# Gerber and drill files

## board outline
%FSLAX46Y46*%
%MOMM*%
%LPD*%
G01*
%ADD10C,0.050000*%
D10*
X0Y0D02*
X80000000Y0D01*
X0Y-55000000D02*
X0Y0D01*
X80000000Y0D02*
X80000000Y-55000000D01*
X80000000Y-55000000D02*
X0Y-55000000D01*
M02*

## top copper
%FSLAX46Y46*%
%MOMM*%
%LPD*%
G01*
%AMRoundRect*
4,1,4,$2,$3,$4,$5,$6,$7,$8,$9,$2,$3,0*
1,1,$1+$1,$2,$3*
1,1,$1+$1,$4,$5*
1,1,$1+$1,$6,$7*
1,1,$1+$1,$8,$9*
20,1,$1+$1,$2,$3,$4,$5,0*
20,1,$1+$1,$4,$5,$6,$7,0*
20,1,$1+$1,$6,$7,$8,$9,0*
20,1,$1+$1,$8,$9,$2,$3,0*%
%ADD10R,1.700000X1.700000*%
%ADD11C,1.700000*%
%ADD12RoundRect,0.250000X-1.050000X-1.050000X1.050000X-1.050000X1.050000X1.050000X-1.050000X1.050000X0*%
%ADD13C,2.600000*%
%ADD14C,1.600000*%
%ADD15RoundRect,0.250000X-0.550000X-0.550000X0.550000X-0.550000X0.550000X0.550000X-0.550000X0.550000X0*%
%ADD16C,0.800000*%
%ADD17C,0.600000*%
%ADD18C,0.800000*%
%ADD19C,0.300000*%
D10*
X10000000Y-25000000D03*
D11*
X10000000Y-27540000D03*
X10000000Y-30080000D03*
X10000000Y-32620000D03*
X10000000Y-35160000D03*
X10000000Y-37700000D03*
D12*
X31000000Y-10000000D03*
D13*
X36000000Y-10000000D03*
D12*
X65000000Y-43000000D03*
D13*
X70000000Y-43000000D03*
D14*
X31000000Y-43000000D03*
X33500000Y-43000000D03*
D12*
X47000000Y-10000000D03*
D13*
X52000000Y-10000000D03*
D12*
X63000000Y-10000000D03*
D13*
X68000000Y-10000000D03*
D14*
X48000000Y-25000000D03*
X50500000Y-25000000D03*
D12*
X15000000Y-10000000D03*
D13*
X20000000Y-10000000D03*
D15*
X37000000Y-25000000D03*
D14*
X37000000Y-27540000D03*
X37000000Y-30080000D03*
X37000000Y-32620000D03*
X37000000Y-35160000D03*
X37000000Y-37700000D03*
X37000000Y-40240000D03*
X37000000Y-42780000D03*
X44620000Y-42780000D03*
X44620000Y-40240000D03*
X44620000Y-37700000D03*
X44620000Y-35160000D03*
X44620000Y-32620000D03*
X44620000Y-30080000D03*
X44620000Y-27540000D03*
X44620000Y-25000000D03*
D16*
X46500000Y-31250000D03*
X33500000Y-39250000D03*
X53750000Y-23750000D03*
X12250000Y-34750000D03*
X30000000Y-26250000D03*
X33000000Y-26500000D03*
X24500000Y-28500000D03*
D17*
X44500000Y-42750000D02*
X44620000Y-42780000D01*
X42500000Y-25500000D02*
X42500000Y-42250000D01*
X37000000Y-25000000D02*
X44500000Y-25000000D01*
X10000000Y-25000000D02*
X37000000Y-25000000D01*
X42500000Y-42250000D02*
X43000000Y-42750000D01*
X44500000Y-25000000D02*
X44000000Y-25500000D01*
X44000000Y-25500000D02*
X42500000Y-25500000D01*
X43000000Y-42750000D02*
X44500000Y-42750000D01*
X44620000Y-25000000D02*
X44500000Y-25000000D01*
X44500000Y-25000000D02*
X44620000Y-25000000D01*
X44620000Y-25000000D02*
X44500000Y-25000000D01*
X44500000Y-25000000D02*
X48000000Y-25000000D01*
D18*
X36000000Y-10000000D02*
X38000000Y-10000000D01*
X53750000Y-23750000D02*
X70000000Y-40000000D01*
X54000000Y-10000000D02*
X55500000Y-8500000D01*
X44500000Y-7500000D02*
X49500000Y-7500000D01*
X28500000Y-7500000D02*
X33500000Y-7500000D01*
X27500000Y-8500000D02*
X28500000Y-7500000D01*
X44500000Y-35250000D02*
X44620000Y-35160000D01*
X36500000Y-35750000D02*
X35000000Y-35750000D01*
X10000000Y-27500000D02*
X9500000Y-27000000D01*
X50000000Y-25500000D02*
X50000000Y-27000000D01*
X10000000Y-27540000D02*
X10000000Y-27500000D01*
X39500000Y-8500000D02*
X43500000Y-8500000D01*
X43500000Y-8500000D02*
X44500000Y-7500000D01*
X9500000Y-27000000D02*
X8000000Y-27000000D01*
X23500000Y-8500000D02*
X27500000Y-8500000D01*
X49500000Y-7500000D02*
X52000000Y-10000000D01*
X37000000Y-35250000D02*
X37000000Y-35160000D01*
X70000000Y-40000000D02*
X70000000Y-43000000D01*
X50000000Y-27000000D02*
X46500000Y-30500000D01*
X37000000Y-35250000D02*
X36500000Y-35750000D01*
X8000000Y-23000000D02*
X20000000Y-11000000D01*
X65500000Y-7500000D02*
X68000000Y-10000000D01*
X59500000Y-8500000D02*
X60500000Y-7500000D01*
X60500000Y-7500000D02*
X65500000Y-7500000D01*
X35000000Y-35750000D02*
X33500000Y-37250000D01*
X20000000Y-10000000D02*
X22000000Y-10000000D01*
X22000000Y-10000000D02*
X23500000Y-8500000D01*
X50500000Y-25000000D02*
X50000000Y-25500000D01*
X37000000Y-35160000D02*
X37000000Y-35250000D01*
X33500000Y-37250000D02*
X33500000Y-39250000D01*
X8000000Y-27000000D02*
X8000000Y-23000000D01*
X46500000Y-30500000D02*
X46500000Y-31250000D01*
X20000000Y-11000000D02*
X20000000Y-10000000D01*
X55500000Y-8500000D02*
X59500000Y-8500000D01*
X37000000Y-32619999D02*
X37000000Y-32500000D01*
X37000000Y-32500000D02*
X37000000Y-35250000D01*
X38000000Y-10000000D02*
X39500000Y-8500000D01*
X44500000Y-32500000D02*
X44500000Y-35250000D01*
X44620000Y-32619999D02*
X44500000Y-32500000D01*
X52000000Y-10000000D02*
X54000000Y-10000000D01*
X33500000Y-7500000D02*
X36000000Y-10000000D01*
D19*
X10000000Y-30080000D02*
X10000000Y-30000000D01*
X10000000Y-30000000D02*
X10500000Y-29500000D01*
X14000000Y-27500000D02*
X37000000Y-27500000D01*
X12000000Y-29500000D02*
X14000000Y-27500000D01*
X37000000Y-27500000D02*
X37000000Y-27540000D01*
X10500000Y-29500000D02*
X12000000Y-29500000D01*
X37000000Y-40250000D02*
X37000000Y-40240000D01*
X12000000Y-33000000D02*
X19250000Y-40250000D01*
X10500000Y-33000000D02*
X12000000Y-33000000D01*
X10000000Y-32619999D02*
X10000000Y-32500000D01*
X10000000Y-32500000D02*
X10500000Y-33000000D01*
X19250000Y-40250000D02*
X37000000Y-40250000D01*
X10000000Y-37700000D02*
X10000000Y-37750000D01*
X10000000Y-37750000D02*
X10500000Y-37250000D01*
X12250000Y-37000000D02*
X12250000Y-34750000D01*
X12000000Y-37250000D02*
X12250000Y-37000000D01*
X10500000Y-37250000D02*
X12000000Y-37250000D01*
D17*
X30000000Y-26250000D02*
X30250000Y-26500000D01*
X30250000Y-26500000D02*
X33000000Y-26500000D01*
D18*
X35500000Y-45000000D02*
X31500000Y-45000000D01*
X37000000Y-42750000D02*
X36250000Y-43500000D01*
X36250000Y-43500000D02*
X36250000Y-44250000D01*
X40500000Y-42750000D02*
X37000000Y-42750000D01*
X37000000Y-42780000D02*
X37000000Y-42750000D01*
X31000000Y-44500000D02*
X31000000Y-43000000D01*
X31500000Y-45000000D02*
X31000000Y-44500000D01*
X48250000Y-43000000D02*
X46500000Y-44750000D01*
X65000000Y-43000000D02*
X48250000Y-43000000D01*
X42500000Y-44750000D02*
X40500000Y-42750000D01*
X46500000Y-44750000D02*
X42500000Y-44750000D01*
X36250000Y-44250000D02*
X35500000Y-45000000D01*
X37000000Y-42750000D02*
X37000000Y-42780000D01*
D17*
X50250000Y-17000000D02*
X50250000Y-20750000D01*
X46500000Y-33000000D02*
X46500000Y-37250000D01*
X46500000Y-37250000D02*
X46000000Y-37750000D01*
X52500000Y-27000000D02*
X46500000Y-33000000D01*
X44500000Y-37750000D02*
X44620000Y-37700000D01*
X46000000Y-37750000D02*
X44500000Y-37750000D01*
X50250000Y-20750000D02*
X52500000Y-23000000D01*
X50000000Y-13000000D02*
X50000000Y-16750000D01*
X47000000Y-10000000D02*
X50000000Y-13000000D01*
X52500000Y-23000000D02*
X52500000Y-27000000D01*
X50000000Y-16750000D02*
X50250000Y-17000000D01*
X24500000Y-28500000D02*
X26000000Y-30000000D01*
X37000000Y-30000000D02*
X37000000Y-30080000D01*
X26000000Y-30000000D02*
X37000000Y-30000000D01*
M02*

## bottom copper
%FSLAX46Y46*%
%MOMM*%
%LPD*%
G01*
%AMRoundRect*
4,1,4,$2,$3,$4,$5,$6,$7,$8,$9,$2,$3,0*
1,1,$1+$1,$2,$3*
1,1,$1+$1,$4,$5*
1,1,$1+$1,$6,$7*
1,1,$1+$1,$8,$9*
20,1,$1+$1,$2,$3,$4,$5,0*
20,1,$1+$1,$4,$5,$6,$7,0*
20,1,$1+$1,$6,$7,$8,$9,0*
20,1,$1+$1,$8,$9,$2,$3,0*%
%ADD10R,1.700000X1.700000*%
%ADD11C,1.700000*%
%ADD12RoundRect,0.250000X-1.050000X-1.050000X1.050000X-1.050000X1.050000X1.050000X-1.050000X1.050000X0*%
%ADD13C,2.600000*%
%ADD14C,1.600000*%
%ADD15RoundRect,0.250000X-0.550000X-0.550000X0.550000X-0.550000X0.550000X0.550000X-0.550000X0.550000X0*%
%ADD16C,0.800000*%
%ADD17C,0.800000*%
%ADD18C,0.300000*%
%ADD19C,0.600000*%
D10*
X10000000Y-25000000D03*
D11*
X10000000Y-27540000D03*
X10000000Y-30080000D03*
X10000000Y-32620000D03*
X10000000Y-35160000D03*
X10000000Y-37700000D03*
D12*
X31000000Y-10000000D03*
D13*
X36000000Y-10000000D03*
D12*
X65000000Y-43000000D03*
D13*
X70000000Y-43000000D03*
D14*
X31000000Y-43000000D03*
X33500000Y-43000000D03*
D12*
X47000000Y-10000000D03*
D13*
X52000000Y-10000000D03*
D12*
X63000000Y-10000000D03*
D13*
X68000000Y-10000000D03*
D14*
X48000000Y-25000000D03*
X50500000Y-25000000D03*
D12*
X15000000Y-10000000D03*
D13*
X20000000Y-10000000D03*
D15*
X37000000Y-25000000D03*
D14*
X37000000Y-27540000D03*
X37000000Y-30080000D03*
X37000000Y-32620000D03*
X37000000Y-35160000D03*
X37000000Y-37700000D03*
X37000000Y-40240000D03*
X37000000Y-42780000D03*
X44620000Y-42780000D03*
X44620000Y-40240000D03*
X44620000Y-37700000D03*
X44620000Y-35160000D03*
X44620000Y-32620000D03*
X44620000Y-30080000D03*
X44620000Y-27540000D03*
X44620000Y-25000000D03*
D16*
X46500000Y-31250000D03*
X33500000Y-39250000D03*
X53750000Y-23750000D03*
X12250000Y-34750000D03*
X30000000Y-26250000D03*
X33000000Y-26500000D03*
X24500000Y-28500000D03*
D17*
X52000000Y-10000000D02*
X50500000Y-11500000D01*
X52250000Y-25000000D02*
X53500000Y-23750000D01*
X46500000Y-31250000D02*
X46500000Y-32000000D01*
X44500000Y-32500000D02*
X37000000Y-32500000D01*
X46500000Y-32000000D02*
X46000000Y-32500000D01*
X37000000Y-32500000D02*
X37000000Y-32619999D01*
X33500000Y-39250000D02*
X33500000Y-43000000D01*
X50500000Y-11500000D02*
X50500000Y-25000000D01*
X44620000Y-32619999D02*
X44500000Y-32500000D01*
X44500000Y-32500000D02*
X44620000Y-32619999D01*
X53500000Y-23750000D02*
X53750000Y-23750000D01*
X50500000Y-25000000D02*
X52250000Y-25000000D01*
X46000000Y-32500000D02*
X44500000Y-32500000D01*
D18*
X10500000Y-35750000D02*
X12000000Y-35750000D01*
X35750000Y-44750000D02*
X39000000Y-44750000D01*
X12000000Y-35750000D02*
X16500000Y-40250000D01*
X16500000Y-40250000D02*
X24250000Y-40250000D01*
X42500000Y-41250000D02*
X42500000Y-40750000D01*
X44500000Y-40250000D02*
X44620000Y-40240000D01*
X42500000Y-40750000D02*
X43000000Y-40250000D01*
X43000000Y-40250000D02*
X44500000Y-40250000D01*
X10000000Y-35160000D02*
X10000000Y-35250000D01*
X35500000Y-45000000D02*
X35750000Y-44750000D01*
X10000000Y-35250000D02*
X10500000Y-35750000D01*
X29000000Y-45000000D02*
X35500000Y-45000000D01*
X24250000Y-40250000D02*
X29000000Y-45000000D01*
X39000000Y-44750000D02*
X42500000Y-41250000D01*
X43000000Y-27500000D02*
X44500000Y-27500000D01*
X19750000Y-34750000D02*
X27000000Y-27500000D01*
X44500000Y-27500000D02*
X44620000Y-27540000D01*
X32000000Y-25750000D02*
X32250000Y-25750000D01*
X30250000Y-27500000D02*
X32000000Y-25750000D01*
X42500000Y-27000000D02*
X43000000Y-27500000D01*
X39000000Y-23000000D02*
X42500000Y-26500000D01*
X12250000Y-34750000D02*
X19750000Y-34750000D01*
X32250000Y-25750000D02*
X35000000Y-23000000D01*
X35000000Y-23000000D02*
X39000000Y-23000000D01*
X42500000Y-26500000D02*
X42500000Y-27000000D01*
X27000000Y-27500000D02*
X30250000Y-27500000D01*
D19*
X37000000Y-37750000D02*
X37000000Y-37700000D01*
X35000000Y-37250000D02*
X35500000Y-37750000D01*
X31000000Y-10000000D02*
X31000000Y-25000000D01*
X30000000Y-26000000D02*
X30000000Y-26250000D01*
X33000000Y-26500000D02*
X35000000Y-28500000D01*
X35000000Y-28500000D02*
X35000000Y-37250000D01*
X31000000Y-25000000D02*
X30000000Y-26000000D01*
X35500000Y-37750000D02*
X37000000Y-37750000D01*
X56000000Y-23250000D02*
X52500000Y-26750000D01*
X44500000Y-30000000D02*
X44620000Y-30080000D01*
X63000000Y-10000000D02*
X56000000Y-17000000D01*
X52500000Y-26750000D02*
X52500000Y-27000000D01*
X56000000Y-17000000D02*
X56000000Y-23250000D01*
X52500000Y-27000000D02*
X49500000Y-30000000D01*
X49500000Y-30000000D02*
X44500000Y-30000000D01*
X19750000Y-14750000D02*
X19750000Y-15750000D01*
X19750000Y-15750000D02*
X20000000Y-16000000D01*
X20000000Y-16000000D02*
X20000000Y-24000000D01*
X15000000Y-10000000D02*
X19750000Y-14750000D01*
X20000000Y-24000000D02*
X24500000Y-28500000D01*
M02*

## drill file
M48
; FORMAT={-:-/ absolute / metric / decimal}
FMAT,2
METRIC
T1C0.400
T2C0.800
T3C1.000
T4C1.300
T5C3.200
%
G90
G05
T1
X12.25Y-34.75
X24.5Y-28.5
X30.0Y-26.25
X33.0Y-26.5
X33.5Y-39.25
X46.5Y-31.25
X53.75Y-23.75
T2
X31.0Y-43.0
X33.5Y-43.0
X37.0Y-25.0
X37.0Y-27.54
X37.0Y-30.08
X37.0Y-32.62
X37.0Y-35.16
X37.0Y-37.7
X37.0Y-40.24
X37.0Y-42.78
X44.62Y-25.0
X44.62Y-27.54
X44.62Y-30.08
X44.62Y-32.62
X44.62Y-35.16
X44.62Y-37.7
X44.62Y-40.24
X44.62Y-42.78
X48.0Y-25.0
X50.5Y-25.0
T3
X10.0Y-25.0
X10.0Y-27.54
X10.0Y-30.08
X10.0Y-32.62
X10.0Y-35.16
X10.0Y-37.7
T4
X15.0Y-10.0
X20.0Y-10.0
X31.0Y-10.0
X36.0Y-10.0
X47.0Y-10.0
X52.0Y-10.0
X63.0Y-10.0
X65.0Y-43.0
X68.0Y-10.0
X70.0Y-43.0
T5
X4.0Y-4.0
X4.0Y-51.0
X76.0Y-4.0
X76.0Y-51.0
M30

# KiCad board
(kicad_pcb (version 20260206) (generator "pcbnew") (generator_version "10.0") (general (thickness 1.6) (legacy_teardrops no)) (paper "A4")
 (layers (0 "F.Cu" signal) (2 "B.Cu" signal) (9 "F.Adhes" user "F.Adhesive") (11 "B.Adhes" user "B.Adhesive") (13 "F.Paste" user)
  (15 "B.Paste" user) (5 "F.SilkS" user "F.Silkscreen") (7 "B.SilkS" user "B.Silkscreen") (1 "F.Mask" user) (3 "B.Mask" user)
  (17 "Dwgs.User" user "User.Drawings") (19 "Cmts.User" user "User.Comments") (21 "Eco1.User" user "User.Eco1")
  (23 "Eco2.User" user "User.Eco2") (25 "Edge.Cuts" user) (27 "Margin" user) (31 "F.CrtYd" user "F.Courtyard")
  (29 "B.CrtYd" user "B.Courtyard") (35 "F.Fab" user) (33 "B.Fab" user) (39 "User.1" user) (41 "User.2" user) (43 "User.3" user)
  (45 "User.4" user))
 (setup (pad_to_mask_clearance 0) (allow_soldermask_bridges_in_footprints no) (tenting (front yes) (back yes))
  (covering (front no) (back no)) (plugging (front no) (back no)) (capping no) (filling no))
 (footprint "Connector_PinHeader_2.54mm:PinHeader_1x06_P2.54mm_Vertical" (layer "F.Cu") (at 10 25)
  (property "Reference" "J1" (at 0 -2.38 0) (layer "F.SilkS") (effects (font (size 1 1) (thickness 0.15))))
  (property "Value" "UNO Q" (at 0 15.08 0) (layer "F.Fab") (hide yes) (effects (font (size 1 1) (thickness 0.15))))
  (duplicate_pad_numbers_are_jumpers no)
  (pad "1" thru_hole rect (at 0 0) (size 1.7 1.7) (drill 1) (layers "*.Cu" "*.Mask") (remove_unused_layers no) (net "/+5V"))
  (pad "2" thru_hole circle (at 0 2.54) (size 1.7 1.7) (drill 1) (layers "*.Cu" "*.Mask") (remove_unused_layers no) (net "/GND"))
  (pad "3" thru_hole circle (at 0 5.08) (size 1.7 1.7) (drill 1) (layers "*.Cu" "*.Mask") (remove_unused_layers no) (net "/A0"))
  (pad "4" thru_hole circle (at 0 7.62) (size 1.7 1.7) (drill 1) (layers "*.Cu" "*.Mask") (remove_unused_layers no) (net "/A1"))
  (pad "5" thru_hole circle (at 0 10.16) (size 1.7 1.7) (drill 1) (layers "*.Cu" "*.Mask") (remove_unused_layers no) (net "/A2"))
  (pad "6" thru_hole circle (at 0 12.7) (size 1.7 1.7) (drill 1) (layers "*.Cu" "*.Mask") (remove_unused_layers no) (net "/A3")))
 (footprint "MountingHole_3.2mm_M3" (layer "F.Cu") (at 76 51)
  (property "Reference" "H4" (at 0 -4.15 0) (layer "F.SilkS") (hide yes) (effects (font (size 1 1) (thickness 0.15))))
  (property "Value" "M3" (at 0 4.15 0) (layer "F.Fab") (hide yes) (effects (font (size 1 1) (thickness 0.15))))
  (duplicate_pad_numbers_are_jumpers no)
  (pad "" np_thru_hole circle (at 0 0) (size 3.2 3.2) (drill 3.2) (layers "*.Cu" "*.Mask")))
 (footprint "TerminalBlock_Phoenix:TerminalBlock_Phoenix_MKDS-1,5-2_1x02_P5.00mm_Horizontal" (layer "F.Cu") (at 31 10)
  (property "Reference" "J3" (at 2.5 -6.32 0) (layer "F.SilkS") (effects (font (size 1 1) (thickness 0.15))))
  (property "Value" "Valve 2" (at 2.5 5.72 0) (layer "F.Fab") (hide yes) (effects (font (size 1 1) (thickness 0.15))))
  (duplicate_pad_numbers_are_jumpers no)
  (pad "1" thru_hole roundrect (at 0 0) (size 2.6 2.6) (drill 1.3) (layers "*.Cu" "*.Mask") (remove_unused_layers no)
   (roundrect_rratio 0.096154) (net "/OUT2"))
  (pad "2" thru_hole circle (at 5 0) (size 2.6 2.6) (drill 1.3) (layers "*.Cu" "*.Mask") (remove_unused_layers no) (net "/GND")))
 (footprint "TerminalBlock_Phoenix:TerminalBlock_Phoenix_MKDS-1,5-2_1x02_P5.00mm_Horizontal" (layer "F.Cu") (at 65 43)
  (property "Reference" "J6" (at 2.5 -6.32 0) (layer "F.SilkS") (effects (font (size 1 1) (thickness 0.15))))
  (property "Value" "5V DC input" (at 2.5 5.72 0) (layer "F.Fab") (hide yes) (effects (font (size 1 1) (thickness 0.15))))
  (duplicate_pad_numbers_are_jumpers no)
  (pad "1" thru_hole roundrect (at 0 0) (size 2.6 2.6) (drill 1.3) (layers "*.Cu" "*.Mask") (remove_unused_layers no)
   (roundrect_rratio 0.096154) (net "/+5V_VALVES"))
  (pad "2" thru_hole circle (at 5 0) (size 2.6 2.6) (drill 1.3) (layers "*.Cu" "*.Mask") (remove_unused_layers no) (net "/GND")))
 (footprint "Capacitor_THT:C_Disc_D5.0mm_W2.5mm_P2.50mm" (layer "F.Cu") (at 31 43)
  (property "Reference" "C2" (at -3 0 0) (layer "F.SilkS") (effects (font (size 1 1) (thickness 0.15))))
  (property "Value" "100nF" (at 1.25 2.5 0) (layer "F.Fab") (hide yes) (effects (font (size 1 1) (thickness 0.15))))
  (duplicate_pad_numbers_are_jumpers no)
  (pad "1" thru_hole circle (at 0 0) (size 1.6 1.6) (drill 0.8) (layers "*.Cu" "*.Mask") (remove_unused_layers no) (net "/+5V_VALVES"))
  (pad "2" thru_hole circle (at 2.5 0) (size 1.6 1.6) (drill 0.8) (layers "*.Cu" "*.Mask") (remove_unused_layers no) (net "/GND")))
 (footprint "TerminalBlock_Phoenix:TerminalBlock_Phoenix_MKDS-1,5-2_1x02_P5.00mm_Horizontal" (layer "F.Cu") (at 47 10)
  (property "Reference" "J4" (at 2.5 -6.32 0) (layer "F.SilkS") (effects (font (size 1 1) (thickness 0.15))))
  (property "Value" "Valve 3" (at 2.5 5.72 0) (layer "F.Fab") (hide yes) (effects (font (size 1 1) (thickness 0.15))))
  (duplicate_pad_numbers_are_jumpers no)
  (pad "1" thru_hole roundrect (at 0 0) (size 2.6 2.6) (drill 1.3) (layers "*.Cu" "*.Mask") (remove_unused_layers no)
   (roundrect_rratio 0.096154) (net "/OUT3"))
  (pad "2" thru_hole circle (at 5 0) (size 2.6 2.6) (drill 1.3) (layers "*.Cu" "*.Mask") (remove_unused_layers no) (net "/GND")))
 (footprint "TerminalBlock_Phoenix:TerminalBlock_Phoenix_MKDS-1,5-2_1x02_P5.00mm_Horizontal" (layer "F.Cu") (at 63 10)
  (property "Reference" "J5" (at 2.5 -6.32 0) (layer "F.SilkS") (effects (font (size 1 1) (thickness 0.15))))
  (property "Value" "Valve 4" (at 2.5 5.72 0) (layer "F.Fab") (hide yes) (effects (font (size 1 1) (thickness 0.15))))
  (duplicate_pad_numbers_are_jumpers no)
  (pad "1" thru_hole roundrect (at 0 0) (size 2.6 2.6) (drill 1.3) (layers "*.Cu" "*.Mask") (remove_unused_layers no)
   (roundrect_rratio 0.096154) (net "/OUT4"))
  (pad "2" thru_hole circle (at 5 0) (size 2.6 2.6) (drill 1.3) (layers "*.Cu" "*.Mask") (remove_unused_layers no) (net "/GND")))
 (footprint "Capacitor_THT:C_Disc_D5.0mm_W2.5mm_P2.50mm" (layer "F.Cu") (at 48 25)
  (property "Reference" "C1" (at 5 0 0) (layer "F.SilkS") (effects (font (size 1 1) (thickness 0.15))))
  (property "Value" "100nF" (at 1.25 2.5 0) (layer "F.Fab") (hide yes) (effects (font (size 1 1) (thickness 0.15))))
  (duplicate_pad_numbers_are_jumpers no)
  (pad "1" thru_hole circle (at 0 0) (size 1.6 1.6) (drill 0.8) (layers "*.Cu" "*.Mask") (remove_unused_layers no) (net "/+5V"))
  (pad "2" thru_hole circle (at 2.5 0) (size 1.6 1.6) (drill 0.8) (layers "*.Cu" "*.Mask") (remove_unused_layers no) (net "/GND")))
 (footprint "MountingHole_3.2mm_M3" (layer "F.Cu") (at 76 4)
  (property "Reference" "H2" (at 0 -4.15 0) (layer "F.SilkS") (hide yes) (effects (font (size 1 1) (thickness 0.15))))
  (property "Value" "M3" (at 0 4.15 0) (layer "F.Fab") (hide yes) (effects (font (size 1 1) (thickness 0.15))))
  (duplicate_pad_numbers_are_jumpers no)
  (pad "" np_thru_hole circle (at 0 0) (size 3.2 3.2) (drill 3.2) (layers "*.Cu" "*.Mask")))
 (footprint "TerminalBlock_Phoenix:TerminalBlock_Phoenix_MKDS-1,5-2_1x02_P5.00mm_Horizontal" (layer "F.Cu") (at 15 10)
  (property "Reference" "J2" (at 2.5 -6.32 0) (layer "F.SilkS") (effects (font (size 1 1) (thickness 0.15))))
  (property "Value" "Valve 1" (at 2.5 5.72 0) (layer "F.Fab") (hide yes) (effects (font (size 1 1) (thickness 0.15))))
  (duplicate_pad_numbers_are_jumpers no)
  (pad "1" thru_hole roundrect (at 0 0) (size 2.6 2.6) (drill 1.3) (layers "*.Cu" "*.Mask") (remove_unused_layers no)
   (roundrect_rratio 0.096154) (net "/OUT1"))
  (pad "2" thru_hole circle (at 5 0) (size 2.6 2.6) (drill 1.3) (layers "*.Cu" "*.Mask") (remove_unused_layers no) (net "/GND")))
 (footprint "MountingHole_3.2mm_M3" (layer "F.Cu") (at 4 51)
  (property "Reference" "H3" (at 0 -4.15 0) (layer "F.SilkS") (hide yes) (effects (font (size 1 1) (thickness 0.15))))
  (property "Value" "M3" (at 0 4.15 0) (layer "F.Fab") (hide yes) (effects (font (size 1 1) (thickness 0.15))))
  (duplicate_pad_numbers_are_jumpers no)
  (pad "" np_thru_hole circle (at 0 0) (size 3.2 3.2) (drill 3.2) (layers "*.Cu" "*.Mask")))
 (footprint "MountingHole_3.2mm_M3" (layer "F.Cu") (at 4 4)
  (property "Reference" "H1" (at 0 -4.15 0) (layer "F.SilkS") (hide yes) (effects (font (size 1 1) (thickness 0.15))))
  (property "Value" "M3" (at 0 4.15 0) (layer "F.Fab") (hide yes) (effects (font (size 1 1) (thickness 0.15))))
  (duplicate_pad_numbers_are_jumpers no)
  (pad "" np_thru_hole circle (at 0 0) (size 3.2 3.2) (drill 3.2) (layers "*.Cu" "*.Mask")))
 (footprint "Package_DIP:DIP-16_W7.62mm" (layer "F.Cu") (at 37 25)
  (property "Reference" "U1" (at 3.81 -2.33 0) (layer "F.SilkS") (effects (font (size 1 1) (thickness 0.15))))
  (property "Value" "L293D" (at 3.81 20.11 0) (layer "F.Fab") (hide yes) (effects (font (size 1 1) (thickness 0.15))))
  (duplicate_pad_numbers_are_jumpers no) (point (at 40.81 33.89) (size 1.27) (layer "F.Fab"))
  (pad "1" thru_hole roundrect (at 0 0) (size 1.6 1.6) (drill 0.8) (layers "*.Cu" "*.Mask") (remove_unused_layers no)
   (roundrect_rratio 0.15625) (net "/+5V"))
  (pad "2" thru_hole circle (at 0 2.54) (size 1.6 1.6) (drill 0.8) (layers "*.Cu" "*.Mask") (remove_unused_layers no) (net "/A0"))
  (pad "3" thru_hole circle (at 0 5.08) (size 1.6 1.6) (drill 0.8) (layers "*.Cu" "*.Mask") (remove_unused_layers no) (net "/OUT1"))
  (pad "4" thru_hole circle (at 0 7.62) (size 1.6 1.6) (drill 0.8) (layers "*.Cu" "*.Mask") (remove_unused_layers no) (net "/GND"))
  (pad "5" thru_hole circle (at 0 10.16) (size 1.6 1.6) (drill 0.8) (layers "*.Cu" "*.Mask") (remove_unused_layers no) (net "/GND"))
  (pad "6" thru_hole circle (at 0 12.7) (size 1.6 1.6) (drill 0.8) (layers "*.Cu" "*.Mask") (remove_unused_layers no) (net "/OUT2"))
  (pad "7" thru_hole circle (at 0 15.24) (size 1.6 1.6) (drill 0.8) (layers "*.Cu" "*.Mask") (remove_unused_layers no) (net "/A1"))
  (pad "8" thru_hole circle (at 0 17.78) (size 1.6 1.6) (drill 0.8) (layers "*.Cu" "*.Mask") (remove_unused_layers no) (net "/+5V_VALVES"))
  (pad "9" thru_hole circle (at 7.62 17.78) (size 1.6 1.6) (drill 0.8) (layers "*.Cu" "*.Mask") (remove_unused_layers no) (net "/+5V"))
  (pad "10" thru_hole circle (at 7.62 15.24) (size 1.6 1.6) (drill 0.8) (layers "*.Cu" "*.Mask") (remove_unused_layers no) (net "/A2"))
  (pad "11" thru_hole circle (at 7.62 12.7) (size 1.6 1.6) (drill 0.8) (layers "*.Cu" "*.Mask") (remove_unused_layers no) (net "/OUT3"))
  (pad "12" thru_hole circle (at 7.62 10.16) (size 1.6 1.6) (drill 0.8) (layers "*.Cu" "*.Mask") (remove_unused_layers no) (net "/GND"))
  (pad "13" thru_hole circle (at 7.62 7.62) (size 1.6 1.6) (drill 0.8) (layers "*.Cu" "*.Mask") (remove_unused_layers no) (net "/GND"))
  (pad "14" thru_hole circle (at 7.62 5.08) (size 1.6 1.6) (drill 0.8) (layers "*.Cu" "*.Mask") (remove_unused_layers no) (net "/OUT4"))
  (pad "15" thru_hole circle (at 7.62 2.54) (size 1.6 1.6) (drill 0.8) (layers "*.Cu" "*.Mask") (remove_unused_layers no) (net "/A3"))
  (pad "16" thru_hole circle (at 7.62 0) (size 1.6 1.6) (drill 0.8) (layers "*.Cu" "*.Mask") (remove_unused_layers no) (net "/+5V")))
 (gr_line (start 0 0) (end 80 0) (stroke (width 0.05) (type default)) (layer "Edge.Cuts"))
 (gr_line (start 0 55) (end 0 0) (stroke (width 0.05) (type default)) (layer "Edge.Cuts"))
 (gr_line (start 80 0) (end 80 55) (stroke (width 0.05) (type default)) (layer "Edge.Cuts"))
 (gr_line (start 80 55) (end 0 55) (stroke (width 0.05) (type default)) (layer "Edge.Cuts"))
 (segment (start 44.5 42.75) (end 44.62 42.78) (width 0.6) (layer "F.Cu") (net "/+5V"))
 (segment (start 42.5 25.5) (end 42.5 42.25) (width 0.6) (layer "F.Cu") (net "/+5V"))
 (segment (start 37 25) (end 44.5 25) (width 0.6) (layer "F.Cu") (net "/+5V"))
 (segment (start 10 25) (end 37 25) (width 0.6) (layer "F.Cu") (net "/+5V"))
 (segment (start 42.5 42.25) (end 43 42.75) (width 0.6) (layer "F.Cu") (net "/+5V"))
 (segment (start 44.5 25) (end 44 25.5) (width 0.6) (layer "F.Cu") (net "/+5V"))
 (segment (start 44 25.5) (end 42.5 25.5) (width 0.6) (layer "F.Cu") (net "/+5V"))
 (segment (start 43 42.75) (end 44.5 42.75) (width 0.6) (layer "F.Cu") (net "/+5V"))
 (segment (start 44.62 25) (end 44.5 25) (width 0.6) (layer "F.Cu") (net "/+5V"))
 (segment (start 44.5 25) (end 44.62 25) (width 0.6) (layer "F.Cu") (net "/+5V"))
 (segment (start 44.62 25) (end 44.5 25) (width 0.6) (layer "F.Cu") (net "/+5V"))
 (segment (start 44.5 25) (end 48 25) (width 0.6) (layer "F.Cu") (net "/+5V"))
 (segment (start 36 10) (end 38 10) (width 0.8) (layer "F.Cu") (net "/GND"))
 (segment (start 53.75 23.75) (end 70 40) (width 0.8) (layer "F.Cu") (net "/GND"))
 (segment (start 54 10) (end 55.5 8.5) (width 0.8) (layer "F.Cu") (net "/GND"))
 (segment (start 44.5 7.5) (end 49.5 7.5) (width 0.8) (layer "F.Cu") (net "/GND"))
 (segment (start 28.5 7.5) (end 33.5 7.5) (width 0.8) (layer "F.Cu") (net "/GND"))
 (segment (start 27.5 8.5) (end 28.5 7.5) (width 0.8) (layer "F.Cu") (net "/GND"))
 (segment (start 44.5 35.25) (end 44.62 35.16) (width 0.8) (layer "F.Cu") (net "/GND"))
 (segment (start 36.5 35.75) (end 35 35.75) (width 0.8) (layer "F.Cu") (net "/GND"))
 (segment (start 10 27.5) (end 9.5 27) (width 0.8) (layer "F.Cu") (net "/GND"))
 (segment (start 50 25.5) (end 50 27) (width 0.8) (layer "F.Cu") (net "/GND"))
 (segment (start 10 27.54) (end 10 27.5) (width 0.8) (layer "F.Cu") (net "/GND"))
 (segment (start 39.5 8.5) (end 43.5 8.5) (width 0.8) (layer "F.Cu") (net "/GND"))
 (segment (start 43.5 8.5) (end 44.5 7.5) (width 0.8) (layer "F.Cu") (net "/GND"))
 (segment (start 9.5 27) (end 8 27) (width 0.8) (layer "F.Cu") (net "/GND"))
 (segment (start 23.5 8.5) (end 27.5 8.5) (width 0.8) (layer "F.Cu") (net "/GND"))
 (segment (start 49.5 7.5) (end 52 10) (width 0.8) (layer "F.Cu") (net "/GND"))
 (segment (start 37 35.25) (end 37 35.16) (width 0.8) (layer "F.Cu") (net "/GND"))
 (segment (start 70 40) (end 70 43) (width 0.8) (layer "F.Cu") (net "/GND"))
 (segment (start 50 27) (end 46.5 30.5) (width 0.8) (layer "F.Cu") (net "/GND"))
 (segment (start 37 35.25) (end 36.5 35.75) (width 0.8) (layer "F.Cu") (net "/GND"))
 (segment (start 8 23) (end 20 11) (width 0.8) (layer "F.Cu") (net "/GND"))
 (segment (start 65.5 7.5) (end 68 10) (width 0.8) (layer "F.Cu") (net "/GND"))
 (segment (start 59.5 8.5) (end 60.5 7.5) (width 0.8) (layer "F.Cu") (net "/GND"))
 (segment (start 60.5 7.5) (end 65.5 7.5) (width 0.8) (layer "F.Cu") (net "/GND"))
 (segment (start 35 35.75) (end 33.5 37.25) (width 0.8) (layer "F.Cu") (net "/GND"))
 (segment (start 20 10) (end 22 10) (width 0.8) (layer "F.Cu") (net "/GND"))
 (segment (start 22 10) (end 23.5 8.5) (width 0.8) (layer "F.Cu") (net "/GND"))
 (segment (start 50.5 25) (end 50 25.5) (width 0.8) (layer "F.Cu") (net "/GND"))
 (segment (start 37 35.16) (end 37 35.25) (width 0.8) (layer "F.Cu") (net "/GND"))
 (segment (start 33.5 37.25) (end 33.5 39.25) (width 0.8) (layer "F.Cu") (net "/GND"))
 (segment (start 8 27) (end 8 23) (width 0.8) (layer "F.Cu") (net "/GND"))
 (segment (start 46.5 30.5) (end 46.5 31.25) (width 0.8) (layer "F.Cu") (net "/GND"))
 (segment (start 20 11) (end 20 10) (width 0.8) (layer "F.Cu") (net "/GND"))
 (segment (start 55.5 8.5) (end 59.5 8.5) (width 0.8) (layer "F.Cu") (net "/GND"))
 (segment (start 37 32.619999) (end 37 32.5) (width 0.8) (layer "F.Cu") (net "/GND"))
 (segment (start 37 32.5) (end 37 35.25) (width 0.8) (layer "F.Cu") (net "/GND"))
 (segment (start 38 10) (end 39.5 8.5) (width 0.8) (layer "F.Cu") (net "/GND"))
 (segment (start 44.5 32.5) (end 44.5 35.25) (width 0.8) (layer "F.Cu") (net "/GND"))
 (segment (start 44.62 32.619999) (end 44.5 32.5) (width 0.8) (layer "F.Cu") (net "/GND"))
 (segment (start 52 10) (end 54 10) (width 0.8) (layer "F.Cu") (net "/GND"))
 (segment (start 33.5 7.5) (end 36 10) (width 0.8) (layer "F.Cu") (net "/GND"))
 (via (at 46.5 31.25) (size 0.8) (drill 0.4) (layers "F.Cu" "B.Cu") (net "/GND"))
 (via (at 33.5 39.25) (size 0.8) (drill 0.4) (layers "F.Cu" "B.Cu") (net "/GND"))
 (via (at 53.75 23.75) (size 0.8) (drill 0.4) (layers "F.Cu" "B.Cu") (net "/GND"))
 (segment (start 52 10) (end 50.5 11.5) (width 0.8) (layer "B.Cu") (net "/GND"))
 (segment (start 52.25 25) (end 53.5 23.75) (width 0.8) (layer "B.Cu") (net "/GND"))
 (segment (start 46.5 31.25) (end 46.5 32) (width 0.8) (layer "B.Cu") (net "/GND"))
 (segment (start 44.5 32.5) (end 37 32.5) (width 0.8) (layer "B.Cu") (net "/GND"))
 (segment (start 46.5 32) (end 46 32.5) (width 0.8) (layer "B.Cu") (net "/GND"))
 (segment (start 37 32.5) (end 37 32.619999) (width 0.8) (layer "B.Cu") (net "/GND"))
 (segment (start 33.5 39.25) (end 33.5 43) (width 0.8) (layer "B.Cu") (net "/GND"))
 (segment (start 50.5 11.5) (end 50.5 25) (width 0.8) (layer "B.Cu") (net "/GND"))
 (segment (start 44.62 32.619999) (end 44.5 32.5) (width 0.8) (layer "B.Cu") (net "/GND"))
 (segment (start 44.5 32.5) (end 44.62 32.619999) (width 0.8) (layer "B.Cu") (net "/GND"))
 (segment (start 53.5 23.75) (end 53.75 23.75) (width 0.8) (layer "B.Cu") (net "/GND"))
 (segment (start 50.5 25) (end 52.25 25) (width 0.8) (layer "B.Cu") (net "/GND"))
 (segment (start 46 32.5) (end 44.5 32.5) (width 0.8) (layer "B.Cu") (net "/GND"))
 (segment (start 10 30.08) (end 10 30) (width 0.3) (layer "F.Cu") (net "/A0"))
 (segment (start 10 30) (end 10.5 29.5) (width 0.3) (layer "F.Cu") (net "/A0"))
 (segment (start 14 27.5) (end 37 27.5) (width 0.3) (layer "F.Cu") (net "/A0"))
 (segment (start 12 29.5) (end 14 27.5) (width 0.3) (layer "F.Cu") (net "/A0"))
 (segment (start 37 27.5) (end 37 27.54) (width 0.3) (layer "F.Cu") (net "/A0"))
 (segment (start 10.5 29.5) (end 12 29.5) (width 0.3) (layer "F.Cu") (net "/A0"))
 (segment (start 37 40.25) (end 37 40.24) (width 0.3) (layer "F.Cu") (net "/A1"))
 (segment (start 12 33) (end 19.25 40.25) (width 0.3) (layer "F.Cu") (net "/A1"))
 (segment (start 10.5 33) (end 12 33) (width 0.3) (layer "F.Cu") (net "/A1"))
 (segment (start 10 32.619999) (end 10 32.5) (width 0.3) (layer "F.Cu") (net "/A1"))
 (segment (start 10 32.5) (end 10.5 33) (width 0.3) (layer "F.Cu") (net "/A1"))
 (segment (start 19.25 40.25) (end 37 40.25) (width 0.3) (layer "F.Cu") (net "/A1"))
 (segment (start 10.5 35.75) (end 12 35.75) (width 0.3) (layer "B.Cu") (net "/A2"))
 (segment (start 35.75 44.75) (end 39 44.75) (width 0.3) (layer "B.Cu") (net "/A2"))
 (segment (start 12 35.75) (end 16.5 40.25) (width 0.3) (layer "B.Cu") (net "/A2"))
 (segment (start 16.5 40.25) (end 24.25 40.25) (width 0.3) (layer "B.Cu") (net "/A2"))
 (segment (start 42.5 41.25) (end 42.5 40.75) (width 0.3) (layer "B.Cu") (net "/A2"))
 (segment (start 44.5 40.25) (end 44.62 40.24) (width 0.3) (layer "B.Cu") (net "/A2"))
 (segment (start 42.5 40.75) (end 43 40.25) (width 0.3) (layer "B.Cu") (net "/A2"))
 (segment (start 43 40.25) (end 44.5 40.25) (width 0.3) (layer "B.Cu") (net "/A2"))
 (segment (start 10 35.16) (end 10 35.25) (width 0.3) (layer "B.Cu") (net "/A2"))
 (segment (start 35.5 45) (end 35.75 44.75) (width 0.3) (layer "B.Cu") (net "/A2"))
 (segment (start 10 35.25) (end 10.5 35.75) (width 0.3) (layer "B.Cu") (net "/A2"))
 (segment (start 29 45) (end 35.5 45) (width 0.3) (layer "B.Cu") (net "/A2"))
 (segment (start 24.25 40.25) (end 29 45) (width 0.3) (layer "B.Cu") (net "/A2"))
 (segment (start 39 44.75) (end 42.5 41.25) (width 0.3) (layer "B.Cu") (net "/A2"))
 (segment (start 10 37.7) (end 10 37.75) (width 0.3) (layer "F.Cu") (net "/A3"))
 (segment (start 10 37.75) (end 10.5 37.25) (width 0.3) (layer "F.Cu") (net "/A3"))
 (segment (start 12.25 37) (end 12.25 34.75) (width 0.3) (layer "F.Cu") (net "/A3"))
 (segment (start 12 37.25) (end 12.25 37) (width 0.3) (layer "F.Cu") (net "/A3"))
 (segment (start 10.5 37.25) (end 12 37.25) (width 0.3) (layer "F.Cu") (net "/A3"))
 (via (at 12.25 34.75) (size 0.8) (drill 0.4) (layers "F.Cu" "B.Cu") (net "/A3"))
 (segment (start 43 27.5) (end 44.5 27.5) (width 0.3) (layer "B.Cu") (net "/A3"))
 (segment (start 19.75 34.75) (end 27 27.5) (width 0.3) (layer "B.Cu") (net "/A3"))
 (segment (start 44.5 27.5) (end 44.62 27.54) (width 0.3) (layer "B.Cu") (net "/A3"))
 (segment (start 32 25.75) (end 32.25 25.75) (width 0.3) (layer "B.Cu") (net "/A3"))
 (segment (start 30.25 27.5) (end 32 25.75) (width 0.3) (layer "B.Cu") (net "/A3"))
 (segment (start 42.5 27) (end 43 27.5) (width 0.3) (layer "B.Cu") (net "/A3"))
 (segment (start 39 23) (end 42.5 26.5) (width 0.3) (layer "B.Cu") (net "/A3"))
 (segment (start 12.25 34.75) (end 19.75 34.75) (width 0.3) (layer "B.Cu") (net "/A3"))
 (segment (start 32.25 25.75) (end 35 23) (width 0.3) (layer "B.Cu") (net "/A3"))
 (segment (start 35 23) (end 39 23) (width 0.3) (layer "B.Cu") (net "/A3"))
 (segment (start 42.5 26.5) (end 42.5 27) (width 0.3) (layer "B.Cu") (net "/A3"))
 (segment (start 27 27.5) (end 30.25 27.5) (width 0.3) (layer "B.Cu") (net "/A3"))
 (segment (start 30 26.25) (end 30.25 26.5) (width 0.6) (layer "F.Cu") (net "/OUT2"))
 (segment (start 30.25 26.5) (end 33 26.5) (width 0.6) (layer "F.Cu") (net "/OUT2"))
 (via (at 30 26.25) (size 0.8) (drill 0.4) (layers "F.Cu" "B.Cu") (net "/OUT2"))
 (via (at 33 26.5) (size 0.8) (drill 0.4) (layers "F.Cu" "B.Cu") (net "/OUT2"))
 (segment (start 37 37.75) (end 37 37.7) (width 0.6) (layer "B.Cu") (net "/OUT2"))
 (segment (start 35 37.25) (end 35.5 37.75) (width 0.6) (layer "B.Cu") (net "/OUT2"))
 (segment (start 31 10) (end 31 25) (width 0.6) (layer "B.Cu") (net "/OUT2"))
 (segment (start 30 26) (end 30 26.25) (width 0.6) (layer "B.Cu") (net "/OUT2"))
 (segment (start 33 26.5) (end 35 28.5) (width 0.6) (layer "B.Cu") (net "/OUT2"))
 (segment (start 35 28.5) (end 35 37.25) (width 0.6) (layer "B.Cu") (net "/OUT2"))
 (segment (start 31 25) (end 30 26) (width 0.6) (layer "B.Cu") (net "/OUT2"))
 (segment (start 35.5 37.75) (end 37 37.75) (width 0.6) (layer "B.Cu") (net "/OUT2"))
 (segment (start 35.5 45) (end 31.5 45) (width 0.8) (layer "F.Cu") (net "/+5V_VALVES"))
 (segment (start 37 42.75) (end 36.25 43.5) (width 0.8) (layer "F.Cu") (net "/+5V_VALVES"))
 (segment (start 36.25 43.5) (end 36.25 44.25) (width 0.8) (layer "F.Cu") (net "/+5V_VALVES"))
 (segment (start 40.5 42.75) (end 37 42.75) (width 0.8) (layer "F.Cu") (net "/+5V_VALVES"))
 (segment (start 37 42.78) (end 37 42.75) (width 0.8) (layer "F.Cu") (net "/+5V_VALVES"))
 (segment (start 31 44.5) (end 31 43) (width 0.8) (layer "F.Cu") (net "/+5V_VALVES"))
 (segment (start 31.5 45) (end 31 44.5) (width 0.8) (layer "F.Cu") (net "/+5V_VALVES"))
 (segment (start 48.25 43) (end 46.5 44.75) (width 0.8) (layer "F.Cu") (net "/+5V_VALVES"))
 (segment (start 65 43) (end 48.25 43) (width 0.8) (layer "F.Cu") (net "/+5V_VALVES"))
 (segment (start 42.5 44.75) (end 40.5 42.75) (width 0.8) (layer "F.Cu") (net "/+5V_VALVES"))
 (segment (start 46.5 44.75) (end 42.5 44.75) (width 0.8) (layer "F.Cu") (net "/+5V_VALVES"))
 (segment (start 36.25 44.25) (end 35.5 45) (width 0.8) (layer "F.Cu") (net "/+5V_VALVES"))
 (segment (start 37 42.75) (end 37 42.78) (width 0.8) (layer "F.Cu") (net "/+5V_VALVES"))
 (segment (start 50.25 17) (end 50.25 20.75) (width 0.6) (layer "F.Cu") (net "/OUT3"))
 (segment (start 46.5 33) (end 46.5 37.25) (width 0.6) (layer "F.Cu") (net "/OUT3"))
 (segment (start 46.5 37.25) (end 46 37.75) (width 0.6) (layer "F.Cu") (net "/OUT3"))
 (segment (start 52.5 27) (end 46.5 33) (width 0.6) (layer "F.Cu") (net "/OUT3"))
 (segment (start 44.5 37.75) (end 44.62 37.7) (width 0.6) (layer "F.Cu") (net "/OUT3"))
 (segment (start 46 37.75) (end 44.5 37.75) (width 0.6) (layer "F.Cu") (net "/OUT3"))
 (segment (start 50.25 20.75) (end 52.5 23) (width 0.6) (layer "F.Cu") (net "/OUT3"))
 (segment (start 50 13) (end 50 16.75) (width 0.6) (layer "F.Cu") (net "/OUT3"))
 (segment (start 47 10) (end 50 13) (width 0.6) (layer "F.Cu") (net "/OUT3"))
 (segment (start 52.5 23) (end 52.5 27) (width 0.6) (layer "F.Cu") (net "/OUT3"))
 (segment (start 50 16.75) (end 50.25 17) (width 0.6) (layer "F.Cu") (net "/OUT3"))
 (segment (start 56 23.25) (end 52.5 26.75) (width 0.6) (layer "B.Cu") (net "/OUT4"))
 (segment (start 44.5 30) (end 44.62 30.08) (width 0.6) (layer "B.Cu") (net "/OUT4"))
 (segment (start 63 10) (end 56 17) (width 0.6) (layer "B.Cu") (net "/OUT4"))
 (segment (start 52.5 26.75) (end 52.5 27) (width 0.6) (layer "B.Cu") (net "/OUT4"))
 (segment (start 56 17) (end 56 23.25) (width 0.6) (layer "B.Cu") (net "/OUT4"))
 (segment (start 52.5 27) (end 49.5 30) (width 0.6) (layer "B.Cu") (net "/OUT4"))
 (segment (start 49.5 30) (end 44.5 30) (width 0.6) (layer "B.Cu") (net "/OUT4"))
 (segment (start 24.5 28.5) (end 26 30) (width 0.6) (layer "F.Cu") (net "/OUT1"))
 (segment (start 37 30) (end 37 30.08) (width 0.6) (layer "F.Cu") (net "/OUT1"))
 (segment (start 26 30) (end 37 30) (width 0.6) (layer "F.Cu") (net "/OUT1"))
 (via (at 24.5 28.5) (size 0.8) (drill 0.4) (layers "F.Cu" "B.Cu") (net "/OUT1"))
 (segment (start 19.75 14.75) (end 19.75 15.75) (width 0.6) (layer "B.Cu") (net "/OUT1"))
 (segment (start 19.75 15.75) (end 20 16) (width 0.6) (layer "B.Cu") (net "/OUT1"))
 (segment (start 20 16) (end 20 24) (width 0.6) (layer "B.Cu") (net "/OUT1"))
 (segment (start 15 10) (end 19.75 14.75) (width 0.6) (layer "B.Cu") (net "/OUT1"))
 (segment (start 20 24) (end 24.5 28.5) (width 0.6) (layer "B.Cu") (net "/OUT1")))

